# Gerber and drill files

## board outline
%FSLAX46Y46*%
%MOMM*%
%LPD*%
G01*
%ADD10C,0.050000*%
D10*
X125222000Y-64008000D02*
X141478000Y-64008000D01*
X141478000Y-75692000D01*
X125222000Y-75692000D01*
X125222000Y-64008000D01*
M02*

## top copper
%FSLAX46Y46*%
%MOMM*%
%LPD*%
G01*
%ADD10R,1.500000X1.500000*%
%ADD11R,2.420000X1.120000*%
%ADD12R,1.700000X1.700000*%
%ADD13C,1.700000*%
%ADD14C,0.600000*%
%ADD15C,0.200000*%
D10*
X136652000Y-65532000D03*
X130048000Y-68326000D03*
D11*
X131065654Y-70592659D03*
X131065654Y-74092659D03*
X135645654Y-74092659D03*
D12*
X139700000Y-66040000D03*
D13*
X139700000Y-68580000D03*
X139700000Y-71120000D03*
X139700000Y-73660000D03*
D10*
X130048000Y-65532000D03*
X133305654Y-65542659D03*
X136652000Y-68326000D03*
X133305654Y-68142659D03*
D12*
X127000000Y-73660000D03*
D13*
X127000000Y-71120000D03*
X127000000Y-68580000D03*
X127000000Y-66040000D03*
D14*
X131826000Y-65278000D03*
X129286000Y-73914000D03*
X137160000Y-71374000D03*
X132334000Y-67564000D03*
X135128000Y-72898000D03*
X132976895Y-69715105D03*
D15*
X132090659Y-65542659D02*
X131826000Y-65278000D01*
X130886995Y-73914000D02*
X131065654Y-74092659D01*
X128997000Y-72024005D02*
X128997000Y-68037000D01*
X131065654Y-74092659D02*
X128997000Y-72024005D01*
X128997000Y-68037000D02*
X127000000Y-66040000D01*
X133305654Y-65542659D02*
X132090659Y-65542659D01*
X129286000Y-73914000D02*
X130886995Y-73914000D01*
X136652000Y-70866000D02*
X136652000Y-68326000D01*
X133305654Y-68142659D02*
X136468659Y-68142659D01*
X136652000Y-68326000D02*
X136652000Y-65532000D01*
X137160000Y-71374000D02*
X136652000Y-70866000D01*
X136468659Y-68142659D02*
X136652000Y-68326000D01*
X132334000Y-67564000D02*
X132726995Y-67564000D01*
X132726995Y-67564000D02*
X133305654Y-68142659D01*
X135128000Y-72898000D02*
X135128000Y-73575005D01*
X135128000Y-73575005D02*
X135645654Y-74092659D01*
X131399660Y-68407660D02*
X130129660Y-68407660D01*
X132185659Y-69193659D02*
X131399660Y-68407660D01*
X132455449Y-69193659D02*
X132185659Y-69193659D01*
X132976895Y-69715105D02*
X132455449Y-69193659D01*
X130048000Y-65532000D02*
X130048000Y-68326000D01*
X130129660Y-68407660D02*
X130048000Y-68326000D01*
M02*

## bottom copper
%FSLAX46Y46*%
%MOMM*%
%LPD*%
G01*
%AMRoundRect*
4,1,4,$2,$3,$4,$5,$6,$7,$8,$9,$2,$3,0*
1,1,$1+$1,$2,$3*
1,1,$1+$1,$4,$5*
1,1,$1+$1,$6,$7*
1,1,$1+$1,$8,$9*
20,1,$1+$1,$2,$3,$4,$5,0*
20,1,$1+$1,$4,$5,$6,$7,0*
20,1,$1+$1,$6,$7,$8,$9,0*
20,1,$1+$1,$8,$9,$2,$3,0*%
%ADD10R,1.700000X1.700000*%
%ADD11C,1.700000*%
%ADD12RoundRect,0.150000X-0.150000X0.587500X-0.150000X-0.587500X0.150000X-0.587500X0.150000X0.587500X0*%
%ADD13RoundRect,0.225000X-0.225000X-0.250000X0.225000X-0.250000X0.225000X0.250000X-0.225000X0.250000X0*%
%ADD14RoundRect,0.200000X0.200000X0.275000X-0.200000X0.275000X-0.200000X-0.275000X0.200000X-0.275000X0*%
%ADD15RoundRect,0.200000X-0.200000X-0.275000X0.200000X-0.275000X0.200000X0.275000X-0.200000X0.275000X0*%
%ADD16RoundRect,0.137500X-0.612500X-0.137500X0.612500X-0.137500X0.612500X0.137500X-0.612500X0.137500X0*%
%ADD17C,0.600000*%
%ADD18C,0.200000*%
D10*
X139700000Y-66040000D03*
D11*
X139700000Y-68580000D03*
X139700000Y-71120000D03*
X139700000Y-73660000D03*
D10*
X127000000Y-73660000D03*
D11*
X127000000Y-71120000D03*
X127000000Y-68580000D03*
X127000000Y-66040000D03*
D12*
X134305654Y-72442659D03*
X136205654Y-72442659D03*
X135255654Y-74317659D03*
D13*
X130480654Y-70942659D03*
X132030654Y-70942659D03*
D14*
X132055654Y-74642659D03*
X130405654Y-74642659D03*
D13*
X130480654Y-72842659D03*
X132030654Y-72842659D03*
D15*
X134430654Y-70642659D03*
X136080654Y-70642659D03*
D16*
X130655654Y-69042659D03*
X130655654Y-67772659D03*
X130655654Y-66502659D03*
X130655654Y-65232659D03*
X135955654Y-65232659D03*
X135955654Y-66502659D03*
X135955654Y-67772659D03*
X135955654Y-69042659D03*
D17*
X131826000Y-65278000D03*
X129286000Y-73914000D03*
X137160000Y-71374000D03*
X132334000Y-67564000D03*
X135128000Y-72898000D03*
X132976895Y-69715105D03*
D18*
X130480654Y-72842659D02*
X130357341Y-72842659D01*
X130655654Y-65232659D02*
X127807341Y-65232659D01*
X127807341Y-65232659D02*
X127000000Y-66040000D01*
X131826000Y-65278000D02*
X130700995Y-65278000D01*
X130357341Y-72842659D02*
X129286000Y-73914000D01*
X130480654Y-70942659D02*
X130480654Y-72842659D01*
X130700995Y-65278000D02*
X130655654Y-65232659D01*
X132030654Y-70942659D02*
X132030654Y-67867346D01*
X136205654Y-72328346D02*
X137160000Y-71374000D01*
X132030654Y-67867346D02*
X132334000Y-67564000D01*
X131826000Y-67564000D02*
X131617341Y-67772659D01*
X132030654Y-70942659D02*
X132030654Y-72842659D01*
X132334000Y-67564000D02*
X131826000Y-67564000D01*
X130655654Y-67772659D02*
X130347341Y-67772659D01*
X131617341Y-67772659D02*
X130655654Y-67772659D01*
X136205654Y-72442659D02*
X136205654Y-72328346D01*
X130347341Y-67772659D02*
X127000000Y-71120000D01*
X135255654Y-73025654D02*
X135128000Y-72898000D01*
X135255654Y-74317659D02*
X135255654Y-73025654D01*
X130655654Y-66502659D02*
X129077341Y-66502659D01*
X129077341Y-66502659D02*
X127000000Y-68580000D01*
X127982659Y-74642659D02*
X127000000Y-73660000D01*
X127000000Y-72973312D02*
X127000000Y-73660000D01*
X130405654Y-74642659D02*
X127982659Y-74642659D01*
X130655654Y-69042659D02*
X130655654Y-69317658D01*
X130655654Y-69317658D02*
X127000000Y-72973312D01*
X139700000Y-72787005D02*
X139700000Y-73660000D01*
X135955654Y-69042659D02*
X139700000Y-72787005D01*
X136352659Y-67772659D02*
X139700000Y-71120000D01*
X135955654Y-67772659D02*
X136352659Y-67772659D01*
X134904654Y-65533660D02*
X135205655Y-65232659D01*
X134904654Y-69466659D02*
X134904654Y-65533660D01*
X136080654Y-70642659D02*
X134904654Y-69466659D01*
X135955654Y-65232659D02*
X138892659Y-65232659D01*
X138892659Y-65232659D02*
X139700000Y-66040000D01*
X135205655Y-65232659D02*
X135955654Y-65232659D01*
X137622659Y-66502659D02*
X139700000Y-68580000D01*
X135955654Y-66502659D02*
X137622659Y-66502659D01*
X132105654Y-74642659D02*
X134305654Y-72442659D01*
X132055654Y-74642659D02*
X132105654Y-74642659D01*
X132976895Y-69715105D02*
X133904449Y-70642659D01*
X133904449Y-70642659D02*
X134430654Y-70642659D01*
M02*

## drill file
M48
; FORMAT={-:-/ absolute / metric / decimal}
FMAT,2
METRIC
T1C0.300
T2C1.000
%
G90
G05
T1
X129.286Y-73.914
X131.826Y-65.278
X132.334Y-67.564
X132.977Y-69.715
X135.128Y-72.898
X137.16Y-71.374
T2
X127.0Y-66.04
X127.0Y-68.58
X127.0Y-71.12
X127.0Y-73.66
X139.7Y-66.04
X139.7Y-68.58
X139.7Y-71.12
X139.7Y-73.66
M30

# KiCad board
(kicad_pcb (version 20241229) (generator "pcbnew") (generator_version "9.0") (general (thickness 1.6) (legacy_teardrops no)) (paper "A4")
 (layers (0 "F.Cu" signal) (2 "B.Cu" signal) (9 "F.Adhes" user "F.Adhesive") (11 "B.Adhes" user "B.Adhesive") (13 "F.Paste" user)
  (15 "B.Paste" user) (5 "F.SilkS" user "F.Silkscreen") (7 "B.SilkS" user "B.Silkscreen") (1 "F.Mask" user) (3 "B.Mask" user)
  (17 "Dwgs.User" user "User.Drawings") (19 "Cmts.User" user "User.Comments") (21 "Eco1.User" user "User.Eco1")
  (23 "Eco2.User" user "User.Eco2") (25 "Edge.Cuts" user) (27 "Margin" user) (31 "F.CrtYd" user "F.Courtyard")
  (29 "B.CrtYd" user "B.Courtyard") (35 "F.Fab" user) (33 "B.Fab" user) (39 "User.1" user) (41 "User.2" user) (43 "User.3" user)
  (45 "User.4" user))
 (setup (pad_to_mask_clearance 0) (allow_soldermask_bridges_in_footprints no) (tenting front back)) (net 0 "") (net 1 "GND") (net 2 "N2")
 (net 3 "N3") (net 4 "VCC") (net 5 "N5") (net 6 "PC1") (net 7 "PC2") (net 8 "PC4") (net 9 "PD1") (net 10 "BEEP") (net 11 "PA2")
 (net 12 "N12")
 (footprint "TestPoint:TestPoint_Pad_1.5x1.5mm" (layer "F.Cu") (at 136.652 65.532)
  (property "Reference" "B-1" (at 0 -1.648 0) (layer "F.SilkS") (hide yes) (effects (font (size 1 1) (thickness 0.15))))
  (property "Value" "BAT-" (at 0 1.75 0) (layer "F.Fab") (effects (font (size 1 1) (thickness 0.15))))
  (pad "1" smd rect (at 0 0) (size 1.5 1.5) (layers "F.Cu" "F.Mask") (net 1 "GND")))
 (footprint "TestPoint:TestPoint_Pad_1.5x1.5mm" (layer "F.Cu") (at 130.048 68.326)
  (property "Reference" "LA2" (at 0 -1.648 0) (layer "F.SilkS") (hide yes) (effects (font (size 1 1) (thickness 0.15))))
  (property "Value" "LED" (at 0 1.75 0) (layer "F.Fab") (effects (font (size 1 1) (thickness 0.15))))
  (pad "1" smd rect (at 0 0) (size 1.5 1.5) (layers "F.Cu" "F.Mask") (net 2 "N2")))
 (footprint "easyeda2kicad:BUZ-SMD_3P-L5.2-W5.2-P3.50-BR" (layer "F.Cu") (at 133.355654 72.342659 90)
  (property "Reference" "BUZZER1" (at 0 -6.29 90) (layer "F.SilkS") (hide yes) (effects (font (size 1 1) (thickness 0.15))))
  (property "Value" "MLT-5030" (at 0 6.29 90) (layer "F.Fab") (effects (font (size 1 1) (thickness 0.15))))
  (pad "1" smd rect (at 1.75 -2.29 270) (size 1.12 2.42) (layers "F.Cu" "F.Mask" "F.Paste") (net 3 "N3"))
  (pad "2" smd rect (at -1.75 -2.29 270) (size 1.12 2.42) (layers "F.Cu" "F.Mask" "F.Paste") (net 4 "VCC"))
  (pad "3" smd rect (at -1.75 2.29 270) (size 1.12 2.42) (layers "F.Cu" "F.Mask" "F.Paste") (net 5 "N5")))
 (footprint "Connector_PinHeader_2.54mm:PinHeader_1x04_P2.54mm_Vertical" (layer "F.Cu") (at 139.7 66.04)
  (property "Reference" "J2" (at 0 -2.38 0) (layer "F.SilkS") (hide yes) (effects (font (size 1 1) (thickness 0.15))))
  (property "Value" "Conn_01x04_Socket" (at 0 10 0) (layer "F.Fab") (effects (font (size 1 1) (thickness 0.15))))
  (pad "1" thru_hole rect (at 0 0) (size 1.7 1.7) (drill 1) (layers "*.Cu" "*.Mask") (remove_unused_layers no) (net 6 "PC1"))
  (pad "2" thru_hole circle (at 0 2.54) (size 1.7 1.7) (drill 1) (layers "*.Cu" "*.Mask") (remove_unused_layers no) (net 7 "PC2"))
  (pad "3" thru_hole circle (at 0 5.08) (size 1.7 1.7) (drill 1) (layers "*.Cu" "*.Mask") (remove_unused_layers no) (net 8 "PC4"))
  (pad "4" thru_hole circle (at 0 7.62) (size 1.7 1.7) (drill 1) (layers "*.Cu" "*.Mask") (remove_unused_layers no) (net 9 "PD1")))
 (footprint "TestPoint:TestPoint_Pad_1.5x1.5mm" (layer "F.Cu") (at 130.048 65.532)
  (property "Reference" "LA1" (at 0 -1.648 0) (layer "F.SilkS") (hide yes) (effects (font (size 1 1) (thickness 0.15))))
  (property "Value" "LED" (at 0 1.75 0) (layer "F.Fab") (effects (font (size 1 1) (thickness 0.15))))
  (pad "1" smd rect (at 0 0) (size 1.5 1.5) (layers "F.Cu" "F.Mask") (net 2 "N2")))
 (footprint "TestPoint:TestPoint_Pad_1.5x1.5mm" (layer "F.Cu") (at 133.305654 65.542659)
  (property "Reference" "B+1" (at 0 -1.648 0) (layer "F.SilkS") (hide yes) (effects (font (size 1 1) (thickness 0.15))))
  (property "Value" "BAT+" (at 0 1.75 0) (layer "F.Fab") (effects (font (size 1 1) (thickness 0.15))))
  (pad "1" smd rect (at 0 0) (size 1.5 1.5) (layers "F.Cu" "F.Mask") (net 4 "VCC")))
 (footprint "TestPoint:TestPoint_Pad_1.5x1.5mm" (layer "F.Cu") (at 136.652 68.326)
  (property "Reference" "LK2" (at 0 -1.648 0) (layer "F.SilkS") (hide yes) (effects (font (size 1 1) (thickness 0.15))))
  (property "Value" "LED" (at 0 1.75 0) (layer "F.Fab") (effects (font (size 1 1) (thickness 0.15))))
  (pad "1" smd rect (at 0 0) (size 1.5 1.5) (layers "F.Cu" "F.Mask") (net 1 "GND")))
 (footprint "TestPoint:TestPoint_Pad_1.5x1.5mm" (layer "F.Cu") (at 133.305654 68.142659)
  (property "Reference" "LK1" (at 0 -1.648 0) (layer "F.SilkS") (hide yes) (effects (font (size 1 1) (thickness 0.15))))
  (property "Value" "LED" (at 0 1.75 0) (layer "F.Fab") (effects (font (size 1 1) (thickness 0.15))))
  (pad "1" smd rect (at 0 0) (size 1.5 1.5) (layers "F.Cu" "F.Mask") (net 1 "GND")))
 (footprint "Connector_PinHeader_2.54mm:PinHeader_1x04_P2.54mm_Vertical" (layer "F.Cu") (at 127 73.66 180)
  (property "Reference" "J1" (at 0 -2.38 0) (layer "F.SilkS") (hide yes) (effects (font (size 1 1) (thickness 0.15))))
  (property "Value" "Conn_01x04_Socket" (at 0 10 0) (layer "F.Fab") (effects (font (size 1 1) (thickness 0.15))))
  (pad "1" thru_hole rect (at 0 0 180) (size 1.7 1.7) (drill 1) (layers "*.Cu" "*.Mask") (remove_unused_layers no) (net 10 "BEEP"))
  (pad "2" thru_hole circle (at 0 2.54 180) (size 1.7 1.7) (drill 1) (layers "*.Cu" "*.Mask") (remove_unused_layers no) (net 1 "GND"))
  (pad "3" thru_hole circle (at 0 5.08 180) (size 1.7 1.7) (drill 1) (layers "*.Cu" "*.Mask") (remove_unused_layers no) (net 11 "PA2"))
  (pad "4" thru_hole circle (at 0 7.62 180) (size 1.7 1.7) (drill 1) (layers "*.Cu" "*.Mask") (remove_unused_layers no) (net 4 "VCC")))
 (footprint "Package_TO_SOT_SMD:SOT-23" (layer "B.Cu") (at 135.255654 73.380159 -90)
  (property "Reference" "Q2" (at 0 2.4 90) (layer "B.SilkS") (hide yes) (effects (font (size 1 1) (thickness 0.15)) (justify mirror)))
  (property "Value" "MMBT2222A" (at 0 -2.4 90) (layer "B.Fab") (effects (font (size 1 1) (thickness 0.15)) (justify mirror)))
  (pad "1" smd roundrect (at -0.9375 0.95 270) (size 1.475 0.6) (layers "B.Cu" "B.Mask" "B.Paste") (roundrect_rratio 0.25) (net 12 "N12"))
  (pad "2" smd roundrect (at -0.9375 -0.95 270) (size 1.475 0.6) (layers "B.Cu" "B.Mask" "B.Paste") (roundrect_rratio 0.25) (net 1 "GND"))
  (pad "3" smd roundrect (at 0.9375 0 270) (size 1.475 0.6) (layers "B.Cu" "B.Mask" "B.Paste") (roundrect_rratio 0.25) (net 5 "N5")))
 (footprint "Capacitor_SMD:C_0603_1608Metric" (layer "B.Cu") (at 131.255654 70.942659)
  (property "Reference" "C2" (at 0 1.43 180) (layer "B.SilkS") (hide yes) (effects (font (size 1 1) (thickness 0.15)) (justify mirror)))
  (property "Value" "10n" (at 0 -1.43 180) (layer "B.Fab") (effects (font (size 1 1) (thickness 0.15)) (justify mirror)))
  (pad "1" smd roundrect (at -0.775 0) (size 0.9 0.95) (layers "B.Cu" "B.Mask" "B.Paste") (roundrect_rratio 0.25) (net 4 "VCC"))
  (pad "2" smd roundrect (at 0.775 0) (size 0.9 0.95) (layers "B.Cu" "B.Mask" "B.Paste") (roundrect_rratio 0.25) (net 1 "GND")))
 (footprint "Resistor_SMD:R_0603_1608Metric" (layer "B.Cu") (at 131.230654 74.642659 180)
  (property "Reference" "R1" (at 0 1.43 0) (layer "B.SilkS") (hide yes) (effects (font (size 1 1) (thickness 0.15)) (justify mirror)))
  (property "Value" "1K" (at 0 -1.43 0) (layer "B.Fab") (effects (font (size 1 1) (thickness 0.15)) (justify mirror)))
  (pad "1" smd roundrect (at -0.825 0 180) (size 0.8 0.95) (layers "B.Cu" "B.Mask" "B.Paste") (roundrect_rratio 0.25) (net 12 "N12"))
  (pad "2" smd roundrect (at 0.825 0 180) (size 0.8 0.95) (layers "B.Cu" "B.Mask" "B.Paste") (roundrect_rratio 0.25) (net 10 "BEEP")))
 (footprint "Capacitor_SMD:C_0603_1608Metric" (layer "B.Cu") (at 131.255654 72.842659)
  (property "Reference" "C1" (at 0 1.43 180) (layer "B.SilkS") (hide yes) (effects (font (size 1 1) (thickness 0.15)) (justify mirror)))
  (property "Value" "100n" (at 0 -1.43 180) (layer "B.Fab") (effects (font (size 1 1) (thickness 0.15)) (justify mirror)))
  (pad "1" smd roundrect (at -0.775 0) (size 0.9 0.95) (layers "B.Cu" "B.Mask" "B.Paste") (roundrect_rratio 0.25) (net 4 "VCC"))
  (pad "2" smd roundrect (at 0.775 0) (size 0.9 0.95) (layers "B.Cu" "B.Mask" "B.Paste") (roundrect_rratio 0.25) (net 1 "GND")))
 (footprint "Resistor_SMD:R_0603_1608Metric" (layer "B.Cu") (at 135.255654 70.642659)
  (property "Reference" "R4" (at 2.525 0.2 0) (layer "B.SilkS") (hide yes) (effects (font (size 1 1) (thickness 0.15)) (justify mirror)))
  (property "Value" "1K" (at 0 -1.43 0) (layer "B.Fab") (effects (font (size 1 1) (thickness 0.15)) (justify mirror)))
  (pad "1" smd roundrect (at -0.825 0) (size 0.8 0.95) (layers "B.Cu" "B.Mask" "B.Paste") (roundrect_rratio 0.25) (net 2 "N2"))
  (pad "2" smd roundrect (at 0.825 0) (size 0.8 0.95) (layers "B.Cu" "B.Mask" "B.Paste") (roundrect_rratio 0.25) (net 6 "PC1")))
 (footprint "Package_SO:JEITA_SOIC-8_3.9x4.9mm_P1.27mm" (layer "B.Cu") (at 133.305654 67.137659)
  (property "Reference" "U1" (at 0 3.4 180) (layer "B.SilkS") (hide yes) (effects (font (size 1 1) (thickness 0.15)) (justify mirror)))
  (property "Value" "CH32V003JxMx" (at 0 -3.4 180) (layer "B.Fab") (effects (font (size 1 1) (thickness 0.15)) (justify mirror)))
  (pad "1" smd roundrect (at -2.65 1.905) (size 1.5 0.55) (layers "B.Cu" "B.Mask" "B.Paste") (roundrect_rratio 0.25) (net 10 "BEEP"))
  (pad "2" smd roundrect (at -2.65 0.635) (size 1.5 0.55) (layers "B.Cu" "B.Mask" "B.Paste") (roundrect_rratio 0.25) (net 1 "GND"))
  (pad "3" smd roundrect (at -2.65 -0.635) (size 1.5 0.55) (layers "B.Cu" "B.Mask" "B.Paste") (roundrect_rratio 0.25) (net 11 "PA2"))
  (pad "4" smd roundrect (at -2.65 -1.905) (size 1.5 0.55) (layers "B.Cu" "B.Mask" "B.Paste") (roundrect_rratio 0.25) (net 4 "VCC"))
  (pad "5" smd roundrect (at 2.65 -1.905) (size 1.5 0.55) (layers "B.Cu" "B.Mask" "B.Paste") (roundrect_rratio 0.25) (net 6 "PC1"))
  (pad "6" smd roundrect (at 2.65 -0.635) (size 1.5 0.55) (layers "B.Cu" "B.Mask" "B.Paste") (roundrect_rratio 0.25) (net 7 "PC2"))
  (pad "7" smd roundrect (at 2.65 0.635) (size 1.5 0.55) (layers "B.Cu" "B.Mask" "B.Paste") (roundrect_rratio 0.25) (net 8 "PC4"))
  (pad "8" smd roundrect (at 2.65 1.905) (size 1.5 0.55) (layers "B.Cu" "B.Mask" "B.Paste") (roundrect_rratio 0.25) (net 9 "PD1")))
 (gr_rect (start 125.222 64.008) (end 141.478 75.692) (stroke (width 0.05) (type default)) (fill no) (layer "Edge.Cuts"))
 (segment (start 132.090659 65.542659) (end 131.826 65.278) (width 0.2) (layer "F.Cu") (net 4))
 (segment (start 130.886995 73.914) (end 131.065654 74.092659) (width 0.2) (layer "F.Cu") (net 4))
 (segment (start 128.997 72.024005) (end 128.997 68.037) (width 0.2) (layer "F.Cu") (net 4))
 (segment (start 131.065654 74.092659) (end 128.997 72.024005) (width 0.2) (layer "F.Cu") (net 4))
 (segment (start 128.997 68.037) (end 127 66.04) (width 0.2) (layer "F.Cu") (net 4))
 (segment (start 133.305654 65.542659) (end 132.090659 65.542659) (width 0.2) (layer "F.Cu") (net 4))
 (segment (start 129.286 73.914) (end 130.886995 73.914) (width 0.2) (layer "F.Cu") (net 4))
 (via (at 131.826 65.278) (size 0.6) (drill 0.3) (layers "F.Cu" "B.Cu") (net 4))
 (via (at 129.286 73.914) (size 0.6) (drill 0.3) (layers "F.Cu" "B.Cu") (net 4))
 (segment (start 130.480654 72.842659) (end 130.357341 72.842659) (width 0.2) (layer "B.Cu") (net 4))
 (segment (start 130.655654 65.232659) (end 127.807341 65.232659) (width 0.2) (layer "B.Cu") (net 4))
 (segment (start 127.807341 65.232659) (end 127 66.04) (width 0.2) (layer "B.Cu") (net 4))
 (segment (start 131.826 65.278) (end 130.700995 65.278) (width 0.2) (layer "B.Cu") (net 4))
 (segment (start 130.357341 72.842659) (end 129.286 73.914) (width 0.2) (layer "B.Cu") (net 4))
 (segment (start 130.480654 70.942659) (end 130.480654 72.842659) (width 0.2) (layer "B.Cu") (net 4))
 (segment (start 130.700995 65.278) (end 130.655654 65.232659) (width 0.2) (layer "B.Cu") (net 4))
 (segment (start 136.652 70.866) (end 136.652 68.326) (width 0.2) (layer "F.Cu") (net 1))
 (segment (start 133.305654 68.142659) (end 136.468659 68.142659) (width 0.2) (layer "F.Cu") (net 1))
 (segment (start 136.652 68.326) (end 136.652 65.532) (width 0.2) (layer "F.Cu") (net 1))
 (segment (start 137.16 71.374) (end 136.652 70.866) (width 0.2) (layer "F.Cu") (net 1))
 (segment (start 136.468659 68.142659) (end 136.652 68.326) (width 0.2) (layer "F.Cu") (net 1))
 (segment (start 132.334 67.564) (end 132.726995 67.564) (width 0.2) (layer "F.Cu") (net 1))
 (segment (start 132.726995 67.564) (end 133.305654 68.142659) (width 0.2) (layer "F.Cu") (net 1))
 (via (at 137.16 71.374) (size 0.6) (drill 0.3) (layers "F.Cu" "B.Cu") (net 1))
 (via (at 132.334 67.564) (size 0.6) (drill 0.3) (layers "F.Cu" "B.Cu") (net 1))
 (segment (start 132.030654 70.942659) (end 132.030654 67.867346) (width 0.2) (layer "B.Cu") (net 1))
 (segment (start 136.205654 72.328346) (end 137.16 71.374) (width 0.2) (layer "B.Cu") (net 1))
 (segment (start 132.030654 67.867346) (end 132.334 67.564) (width 0.2) (layer "B.Cu") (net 1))
 (segment (start 131.826 67.564) (end 131.617341 67.772659) (width 0.2) (layer "B.Cu") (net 1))
 (segment (start 132.030654 70.942659) (end 132.030654 72.842659) (width 0.2) (layer "B.Cu") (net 1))
 (segment (start 132.334 67.564) (end 131.826 67.564) (width 0.2) (layer "B.Cu") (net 1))
 (segment (start 130.655654 67.772659) (end 130.347341 67.772659) (width 0.2) (layer "B.Cu") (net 1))
 (segment (start 131.617341 67.772659) (end 130.655654 67.772659) (width 0.2) (layer "B.Cu") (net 1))
 (segment (start 136.205654 72.442659) (end 136.205654 72.328346) (width 0.2) (layer "B.Cu") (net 1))
 (segment (start 130.347341 67.772659) (end 127 71.12) (width 0.2) (layer "B.Cu") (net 1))
 (segment (start 135.128 72.898) (end 135.128 73.575005) (width 0.2) (layer "F.Cu") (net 5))
 (segment (start 135.128 73.575005) (end 135.645654 74.092659) (width 0.2) (layer "F.Cu") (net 5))
 (via (at 135.128 72.898) (size 0.6) (drill 0.3) (layers "F.Cu" "B.Cu") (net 5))
 (segment (start 135.255654 73.025654) (end 135.128 72.898) (width 0.2) (layer "B.Cu") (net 5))
 (segment (start 135.255654 74.317659) (end 135.255654 73.025654) (width 0.2) (layer "B.Cu") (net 5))
 (segment (start 130.655654 66.502659) (end 129.077341 66.502659) (width 0.2) (layer "B.Cu") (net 11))
 (segment (start 129.077341 66.502659) (end 127 68.58) (width 0.2) (layer "B.Cu") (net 11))
 (segment (start 127.982659 74.642659) (end 127 73.66) (width 0.2) (layer "B.Cu") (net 10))
 (segment (start 127 72.973312) (end 127 73.66) (width 0.2) (layer "B.Cu") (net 10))
 (segment (start 130.405654 74.642659) (end 127.982659 74.642659) (width 0.2) (layer "B.Cu") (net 10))
 (segment (start 130.655654 69.042659) (end 130.655654 69.317658) (width 0.2) (layer "B.Cu") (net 10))
 (segment (start 130.655654 69.317658) (end 127 72.973312) (width 0.2) (layer "B.Cu") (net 10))
 (segment (start 139.7 72.787005) (end 139.7 73.66) (width 0.2) (layer "B.Cu") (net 9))
 (segment (start 135.955654 69.042659) (end 139.7 72.787005) (width 0.2) (layer "B.Cu") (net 9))
 (segment (start 136.352659 67.772659) (end 139.7 71.12) (width 0.2) (layer "B.Cu") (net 8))
 (segment (start 135.955654 67.772659) (end 136.352659 67.772659) (width 0.2) (layer "B.Cu") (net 8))
 (segment (start 134.904654 65.53366) (end 135.205655 65.232659) (width 0.2) (layer "B.Cu") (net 6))
 (segment (start 134.904654 69.466659) (end 134.904654 65.53366) (width 0.2) (layer "B.Cu") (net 6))
 (segment (start 136.080654 70.642659) (end 134.904654 69.466659) (width 0.2) (layer "B.Cu") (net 6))
 (segment (start 135.955654 65.232659) (end 138.892659 65.232659) (width 0.2) (layer "B.Cu") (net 6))
 (segment (start 138.892659 65.232659) (end 139.7 66.04) (width 0.2) (layer "B.Cu") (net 6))
 (segment (start 135.205655 65.232659) (end 135.955654 65.232659) (width 0.2) (layer "B.Cu") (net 6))
 (segment (start 137.622659 66.502659) (end 139.7 68.58) (width 0.2) (layer "B.Cu") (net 7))
 (segment (start 135.955654 66.502659) (end 137.622659 66.502659) (width 0.2) (layer "B.Cu") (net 7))
 (segment (start 132.105654 74.642659) (end 134.305654 72.442659) (width 0.2) (layer "B.Cu") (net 12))
 (segment (start 132.055654 74.642659) (end 132.105654 74.642659) (width 0.2) (layer "B.Cu") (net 12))
 (segment (start 131.39966 68.40766) (end 130.12966 68.40766) (width 0.2) (layer "F.Cu") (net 2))
 (segment (start 132.185659 69.193659) (end 131.39966 68.40766) (width 0.2) (layer "F.Cu") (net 2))
 (segment (start 132.455449 69.193659) (end 132.185659 69.193659) (width 0.2) (layer "F.Cu") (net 2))
 (segment (start 132.976895 69.715105) (end 132.455449 69.193659) (width 0.2) (layer "F.Cu") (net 2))
 (segment (start 130.048 65.532) (end 130.048 68.326) (width 0.2) (layer "F.Cu") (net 2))
 (segment (start 130.12966 68.40766) (end 130.048 68.326) (width 0.2) (layer "F.Cu") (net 2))
 (via (at 132.976895 69.715105) (size 0.6) (drill 0.3) (layers "F.Cu" "B.Cu") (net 2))
 (segment (start 132.976895 69.715105) (end 133.904449 70.642659) (width 0.2) (layer "B.Cu") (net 2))
 (segment (start 133.904449 70.642659) (end 134.430654 70.642659) (width 0.2) (layer "B.Cu") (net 2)))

